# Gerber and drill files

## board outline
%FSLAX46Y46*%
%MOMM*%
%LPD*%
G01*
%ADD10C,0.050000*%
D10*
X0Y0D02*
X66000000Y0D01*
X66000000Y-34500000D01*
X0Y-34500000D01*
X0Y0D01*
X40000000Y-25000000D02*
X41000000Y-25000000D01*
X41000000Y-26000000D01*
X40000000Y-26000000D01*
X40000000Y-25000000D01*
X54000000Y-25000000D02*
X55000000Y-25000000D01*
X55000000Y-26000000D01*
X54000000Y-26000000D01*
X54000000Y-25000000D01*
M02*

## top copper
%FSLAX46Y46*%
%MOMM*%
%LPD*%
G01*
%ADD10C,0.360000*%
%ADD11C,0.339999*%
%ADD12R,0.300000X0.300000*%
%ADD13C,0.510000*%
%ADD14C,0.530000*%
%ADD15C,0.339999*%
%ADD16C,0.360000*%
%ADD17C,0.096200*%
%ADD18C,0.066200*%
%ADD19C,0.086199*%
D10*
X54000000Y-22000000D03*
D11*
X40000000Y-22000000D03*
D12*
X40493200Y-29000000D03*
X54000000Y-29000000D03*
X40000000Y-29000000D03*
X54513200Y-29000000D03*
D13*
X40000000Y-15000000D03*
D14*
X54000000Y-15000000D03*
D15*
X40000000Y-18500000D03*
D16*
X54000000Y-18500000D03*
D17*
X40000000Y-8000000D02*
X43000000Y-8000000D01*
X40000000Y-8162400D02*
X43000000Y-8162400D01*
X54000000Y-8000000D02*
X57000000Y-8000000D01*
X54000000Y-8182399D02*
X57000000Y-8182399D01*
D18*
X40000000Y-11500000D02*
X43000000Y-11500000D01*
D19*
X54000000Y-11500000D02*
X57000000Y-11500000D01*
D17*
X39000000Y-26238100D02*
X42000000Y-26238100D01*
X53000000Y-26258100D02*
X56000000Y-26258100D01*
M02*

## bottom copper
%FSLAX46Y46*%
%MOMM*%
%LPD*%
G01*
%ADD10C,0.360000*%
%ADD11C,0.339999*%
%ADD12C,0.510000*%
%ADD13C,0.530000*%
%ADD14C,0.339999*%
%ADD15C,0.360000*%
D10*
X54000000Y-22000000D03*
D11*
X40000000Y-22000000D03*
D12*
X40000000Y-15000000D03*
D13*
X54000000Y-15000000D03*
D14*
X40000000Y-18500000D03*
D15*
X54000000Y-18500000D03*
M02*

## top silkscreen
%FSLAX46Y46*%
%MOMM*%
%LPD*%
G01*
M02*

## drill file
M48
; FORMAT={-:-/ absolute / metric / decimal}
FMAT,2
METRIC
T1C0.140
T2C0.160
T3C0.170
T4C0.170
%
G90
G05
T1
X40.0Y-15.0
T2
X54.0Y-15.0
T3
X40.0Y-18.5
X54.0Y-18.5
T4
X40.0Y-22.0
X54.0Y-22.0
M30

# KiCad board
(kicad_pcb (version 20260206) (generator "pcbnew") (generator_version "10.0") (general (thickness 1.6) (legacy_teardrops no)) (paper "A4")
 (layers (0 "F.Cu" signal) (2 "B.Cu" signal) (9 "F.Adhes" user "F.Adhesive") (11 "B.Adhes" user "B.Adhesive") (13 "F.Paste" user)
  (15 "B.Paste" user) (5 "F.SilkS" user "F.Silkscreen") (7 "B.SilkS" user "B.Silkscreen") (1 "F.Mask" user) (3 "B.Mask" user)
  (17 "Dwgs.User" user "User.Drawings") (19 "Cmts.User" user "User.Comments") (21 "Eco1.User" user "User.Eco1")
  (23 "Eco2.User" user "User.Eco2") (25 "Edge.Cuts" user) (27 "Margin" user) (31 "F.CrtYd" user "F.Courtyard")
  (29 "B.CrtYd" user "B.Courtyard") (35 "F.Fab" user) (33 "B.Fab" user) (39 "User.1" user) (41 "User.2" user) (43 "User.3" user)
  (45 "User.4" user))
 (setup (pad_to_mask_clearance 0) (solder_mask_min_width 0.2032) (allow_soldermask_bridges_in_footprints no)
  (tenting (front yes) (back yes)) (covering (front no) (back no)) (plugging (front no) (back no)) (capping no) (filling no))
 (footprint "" (layer "F.Cu") (at 54 22)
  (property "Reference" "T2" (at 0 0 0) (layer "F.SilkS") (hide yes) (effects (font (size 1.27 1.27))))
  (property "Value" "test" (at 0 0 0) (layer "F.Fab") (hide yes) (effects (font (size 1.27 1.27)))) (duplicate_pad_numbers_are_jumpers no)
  (pad "1" thru_hole circle (at 0 0) (size 0.36 0.36) (drill 0.169999) (layers "*.Cu" "*.Mask") (remove_unused_layers no) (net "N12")))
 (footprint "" (layer "F.Cu") (at 40 22)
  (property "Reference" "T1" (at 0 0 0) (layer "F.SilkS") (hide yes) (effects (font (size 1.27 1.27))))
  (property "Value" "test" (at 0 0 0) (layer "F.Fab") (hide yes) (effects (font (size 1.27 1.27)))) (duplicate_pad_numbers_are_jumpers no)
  (pad "1" thru_hole circle (at 0 0) (size 0.339999 0.339999) (drill 0.169999) (layers "*.Cu" "*.Mask") (remove_unused_layers no)
   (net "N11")))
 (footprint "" (layer "F.Cu") (at 40.4932 29)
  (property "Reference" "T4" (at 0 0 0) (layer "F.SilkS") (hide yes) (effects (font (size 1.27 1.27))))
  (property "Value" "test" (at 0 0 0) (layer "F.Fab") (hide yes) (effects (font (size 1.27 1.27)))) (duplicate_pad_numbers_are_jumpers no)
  (pad "1" smd rect (at 0 0) (size 0.3 0.3) (layers "F.Cu" "F.Mask" "F.Paste") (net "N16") (thermal_bridge_angle 45)))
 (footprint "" (layer "F.Cu") (at 54 29)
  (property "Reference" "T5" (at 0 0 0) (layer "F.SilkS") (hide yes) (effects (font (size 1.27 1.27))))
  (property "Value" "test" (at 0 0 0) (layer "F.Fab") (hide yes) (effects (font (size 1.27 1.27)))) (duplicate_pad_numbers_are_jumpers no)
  (pad "1" smd rect (at 0 0) (size 0.3 0.3) (layers "F.Cu" "F.Mask" "F.Paste") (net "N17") (thermal_bridge_angle 45)))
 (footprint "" (layer "F.Cu") (at 40 29)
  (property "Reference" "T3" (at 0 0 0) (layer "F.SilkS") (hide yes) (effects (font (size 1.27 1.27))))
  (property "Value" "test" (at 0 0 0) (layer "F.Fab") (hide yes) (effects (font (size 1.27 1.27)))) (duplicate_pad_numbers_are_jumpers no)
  (pad "1" smd rect (at 0 0) (size 0.3 0.3) (layers "F.Cu" "F.Mask" "F.Paste") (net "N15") (thermal_bridge_angle 45)))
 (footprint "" (layer "F.Cu") (at 54.5132 29)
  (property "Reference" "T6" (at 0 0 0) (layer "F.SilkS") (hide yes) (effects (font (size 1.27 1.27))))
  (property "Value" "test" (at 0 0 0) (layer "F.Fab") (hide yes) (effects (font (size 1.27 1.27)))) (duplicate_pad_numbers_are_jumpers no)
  (pad "1" smd rect (at 0 0) (size 0.3 0.3) (layers "F.Cu" "F.Mask" "F.Paste") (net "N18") (thermal_bridge_angle 45)))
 (gr_rect (start 0 0) (end 66 34.5) (stroke (width 0.05) (type default)) (fill no) (layer "Edge.Cuts"))
 (gr_rect (start 40 25) (end 41 26) (stroke (width 0.05) (type default)) (fill no) (layer "Edge.Cuts"))
 (gr_rect (start 54 25) (end 55 26) (stroke (width 0.05) (type default)) (fill no) (layer "Edge.Cuts"))
 (segment (start 40 8) (end 43 8) (width 0.0962) (layer "F.Cu") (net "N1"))
 (segment (start 40 8.1624) (end 43 8.1624) (width 0.0962) (layer "F.Cu") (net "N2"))
 (segment (start 54 8) (end 57 8) (width 0.0962) (layer "F.Cu") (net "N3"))
 (segment (start 54 8.182399) (end 57 8.182399) (width 0.0962) (layer "F.Cu") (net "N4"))
 (segment (start 40 11.5) (end 43 11.5) (width 0.0662) (layer "F.Cu") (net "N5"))
 (segment (start 54 11.5) (end 57 11.5) (width 0.086199) (layer "F.Cu") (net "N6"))
 (via (at 40 15) (size 0.51) (drill 0.14) (layers "F.Cu" "B.Cu") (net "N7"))
 (via (at 54 15) (size 0.53) (drill 0.16) (layers "F.Cu" "B.Cu") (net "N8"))
 (via (at 40 18.5) (size 0.339999) (drill 0.169999) (layers "F.Cu" "B.Cu") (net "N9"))
 (via (at 54 18.5) (size 0.36) (drill 0.169999) (layers "F.Cu" "B.Cu") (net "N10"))
 (segment (start 39 26.2381) (end 42 26.2381) (width 0.0962) (layer "F.Cu") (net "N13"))
 (segment (start 53 26.2581) (end 56 26.2581) (width 0.0962) (layer "F.Cu") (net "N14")))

